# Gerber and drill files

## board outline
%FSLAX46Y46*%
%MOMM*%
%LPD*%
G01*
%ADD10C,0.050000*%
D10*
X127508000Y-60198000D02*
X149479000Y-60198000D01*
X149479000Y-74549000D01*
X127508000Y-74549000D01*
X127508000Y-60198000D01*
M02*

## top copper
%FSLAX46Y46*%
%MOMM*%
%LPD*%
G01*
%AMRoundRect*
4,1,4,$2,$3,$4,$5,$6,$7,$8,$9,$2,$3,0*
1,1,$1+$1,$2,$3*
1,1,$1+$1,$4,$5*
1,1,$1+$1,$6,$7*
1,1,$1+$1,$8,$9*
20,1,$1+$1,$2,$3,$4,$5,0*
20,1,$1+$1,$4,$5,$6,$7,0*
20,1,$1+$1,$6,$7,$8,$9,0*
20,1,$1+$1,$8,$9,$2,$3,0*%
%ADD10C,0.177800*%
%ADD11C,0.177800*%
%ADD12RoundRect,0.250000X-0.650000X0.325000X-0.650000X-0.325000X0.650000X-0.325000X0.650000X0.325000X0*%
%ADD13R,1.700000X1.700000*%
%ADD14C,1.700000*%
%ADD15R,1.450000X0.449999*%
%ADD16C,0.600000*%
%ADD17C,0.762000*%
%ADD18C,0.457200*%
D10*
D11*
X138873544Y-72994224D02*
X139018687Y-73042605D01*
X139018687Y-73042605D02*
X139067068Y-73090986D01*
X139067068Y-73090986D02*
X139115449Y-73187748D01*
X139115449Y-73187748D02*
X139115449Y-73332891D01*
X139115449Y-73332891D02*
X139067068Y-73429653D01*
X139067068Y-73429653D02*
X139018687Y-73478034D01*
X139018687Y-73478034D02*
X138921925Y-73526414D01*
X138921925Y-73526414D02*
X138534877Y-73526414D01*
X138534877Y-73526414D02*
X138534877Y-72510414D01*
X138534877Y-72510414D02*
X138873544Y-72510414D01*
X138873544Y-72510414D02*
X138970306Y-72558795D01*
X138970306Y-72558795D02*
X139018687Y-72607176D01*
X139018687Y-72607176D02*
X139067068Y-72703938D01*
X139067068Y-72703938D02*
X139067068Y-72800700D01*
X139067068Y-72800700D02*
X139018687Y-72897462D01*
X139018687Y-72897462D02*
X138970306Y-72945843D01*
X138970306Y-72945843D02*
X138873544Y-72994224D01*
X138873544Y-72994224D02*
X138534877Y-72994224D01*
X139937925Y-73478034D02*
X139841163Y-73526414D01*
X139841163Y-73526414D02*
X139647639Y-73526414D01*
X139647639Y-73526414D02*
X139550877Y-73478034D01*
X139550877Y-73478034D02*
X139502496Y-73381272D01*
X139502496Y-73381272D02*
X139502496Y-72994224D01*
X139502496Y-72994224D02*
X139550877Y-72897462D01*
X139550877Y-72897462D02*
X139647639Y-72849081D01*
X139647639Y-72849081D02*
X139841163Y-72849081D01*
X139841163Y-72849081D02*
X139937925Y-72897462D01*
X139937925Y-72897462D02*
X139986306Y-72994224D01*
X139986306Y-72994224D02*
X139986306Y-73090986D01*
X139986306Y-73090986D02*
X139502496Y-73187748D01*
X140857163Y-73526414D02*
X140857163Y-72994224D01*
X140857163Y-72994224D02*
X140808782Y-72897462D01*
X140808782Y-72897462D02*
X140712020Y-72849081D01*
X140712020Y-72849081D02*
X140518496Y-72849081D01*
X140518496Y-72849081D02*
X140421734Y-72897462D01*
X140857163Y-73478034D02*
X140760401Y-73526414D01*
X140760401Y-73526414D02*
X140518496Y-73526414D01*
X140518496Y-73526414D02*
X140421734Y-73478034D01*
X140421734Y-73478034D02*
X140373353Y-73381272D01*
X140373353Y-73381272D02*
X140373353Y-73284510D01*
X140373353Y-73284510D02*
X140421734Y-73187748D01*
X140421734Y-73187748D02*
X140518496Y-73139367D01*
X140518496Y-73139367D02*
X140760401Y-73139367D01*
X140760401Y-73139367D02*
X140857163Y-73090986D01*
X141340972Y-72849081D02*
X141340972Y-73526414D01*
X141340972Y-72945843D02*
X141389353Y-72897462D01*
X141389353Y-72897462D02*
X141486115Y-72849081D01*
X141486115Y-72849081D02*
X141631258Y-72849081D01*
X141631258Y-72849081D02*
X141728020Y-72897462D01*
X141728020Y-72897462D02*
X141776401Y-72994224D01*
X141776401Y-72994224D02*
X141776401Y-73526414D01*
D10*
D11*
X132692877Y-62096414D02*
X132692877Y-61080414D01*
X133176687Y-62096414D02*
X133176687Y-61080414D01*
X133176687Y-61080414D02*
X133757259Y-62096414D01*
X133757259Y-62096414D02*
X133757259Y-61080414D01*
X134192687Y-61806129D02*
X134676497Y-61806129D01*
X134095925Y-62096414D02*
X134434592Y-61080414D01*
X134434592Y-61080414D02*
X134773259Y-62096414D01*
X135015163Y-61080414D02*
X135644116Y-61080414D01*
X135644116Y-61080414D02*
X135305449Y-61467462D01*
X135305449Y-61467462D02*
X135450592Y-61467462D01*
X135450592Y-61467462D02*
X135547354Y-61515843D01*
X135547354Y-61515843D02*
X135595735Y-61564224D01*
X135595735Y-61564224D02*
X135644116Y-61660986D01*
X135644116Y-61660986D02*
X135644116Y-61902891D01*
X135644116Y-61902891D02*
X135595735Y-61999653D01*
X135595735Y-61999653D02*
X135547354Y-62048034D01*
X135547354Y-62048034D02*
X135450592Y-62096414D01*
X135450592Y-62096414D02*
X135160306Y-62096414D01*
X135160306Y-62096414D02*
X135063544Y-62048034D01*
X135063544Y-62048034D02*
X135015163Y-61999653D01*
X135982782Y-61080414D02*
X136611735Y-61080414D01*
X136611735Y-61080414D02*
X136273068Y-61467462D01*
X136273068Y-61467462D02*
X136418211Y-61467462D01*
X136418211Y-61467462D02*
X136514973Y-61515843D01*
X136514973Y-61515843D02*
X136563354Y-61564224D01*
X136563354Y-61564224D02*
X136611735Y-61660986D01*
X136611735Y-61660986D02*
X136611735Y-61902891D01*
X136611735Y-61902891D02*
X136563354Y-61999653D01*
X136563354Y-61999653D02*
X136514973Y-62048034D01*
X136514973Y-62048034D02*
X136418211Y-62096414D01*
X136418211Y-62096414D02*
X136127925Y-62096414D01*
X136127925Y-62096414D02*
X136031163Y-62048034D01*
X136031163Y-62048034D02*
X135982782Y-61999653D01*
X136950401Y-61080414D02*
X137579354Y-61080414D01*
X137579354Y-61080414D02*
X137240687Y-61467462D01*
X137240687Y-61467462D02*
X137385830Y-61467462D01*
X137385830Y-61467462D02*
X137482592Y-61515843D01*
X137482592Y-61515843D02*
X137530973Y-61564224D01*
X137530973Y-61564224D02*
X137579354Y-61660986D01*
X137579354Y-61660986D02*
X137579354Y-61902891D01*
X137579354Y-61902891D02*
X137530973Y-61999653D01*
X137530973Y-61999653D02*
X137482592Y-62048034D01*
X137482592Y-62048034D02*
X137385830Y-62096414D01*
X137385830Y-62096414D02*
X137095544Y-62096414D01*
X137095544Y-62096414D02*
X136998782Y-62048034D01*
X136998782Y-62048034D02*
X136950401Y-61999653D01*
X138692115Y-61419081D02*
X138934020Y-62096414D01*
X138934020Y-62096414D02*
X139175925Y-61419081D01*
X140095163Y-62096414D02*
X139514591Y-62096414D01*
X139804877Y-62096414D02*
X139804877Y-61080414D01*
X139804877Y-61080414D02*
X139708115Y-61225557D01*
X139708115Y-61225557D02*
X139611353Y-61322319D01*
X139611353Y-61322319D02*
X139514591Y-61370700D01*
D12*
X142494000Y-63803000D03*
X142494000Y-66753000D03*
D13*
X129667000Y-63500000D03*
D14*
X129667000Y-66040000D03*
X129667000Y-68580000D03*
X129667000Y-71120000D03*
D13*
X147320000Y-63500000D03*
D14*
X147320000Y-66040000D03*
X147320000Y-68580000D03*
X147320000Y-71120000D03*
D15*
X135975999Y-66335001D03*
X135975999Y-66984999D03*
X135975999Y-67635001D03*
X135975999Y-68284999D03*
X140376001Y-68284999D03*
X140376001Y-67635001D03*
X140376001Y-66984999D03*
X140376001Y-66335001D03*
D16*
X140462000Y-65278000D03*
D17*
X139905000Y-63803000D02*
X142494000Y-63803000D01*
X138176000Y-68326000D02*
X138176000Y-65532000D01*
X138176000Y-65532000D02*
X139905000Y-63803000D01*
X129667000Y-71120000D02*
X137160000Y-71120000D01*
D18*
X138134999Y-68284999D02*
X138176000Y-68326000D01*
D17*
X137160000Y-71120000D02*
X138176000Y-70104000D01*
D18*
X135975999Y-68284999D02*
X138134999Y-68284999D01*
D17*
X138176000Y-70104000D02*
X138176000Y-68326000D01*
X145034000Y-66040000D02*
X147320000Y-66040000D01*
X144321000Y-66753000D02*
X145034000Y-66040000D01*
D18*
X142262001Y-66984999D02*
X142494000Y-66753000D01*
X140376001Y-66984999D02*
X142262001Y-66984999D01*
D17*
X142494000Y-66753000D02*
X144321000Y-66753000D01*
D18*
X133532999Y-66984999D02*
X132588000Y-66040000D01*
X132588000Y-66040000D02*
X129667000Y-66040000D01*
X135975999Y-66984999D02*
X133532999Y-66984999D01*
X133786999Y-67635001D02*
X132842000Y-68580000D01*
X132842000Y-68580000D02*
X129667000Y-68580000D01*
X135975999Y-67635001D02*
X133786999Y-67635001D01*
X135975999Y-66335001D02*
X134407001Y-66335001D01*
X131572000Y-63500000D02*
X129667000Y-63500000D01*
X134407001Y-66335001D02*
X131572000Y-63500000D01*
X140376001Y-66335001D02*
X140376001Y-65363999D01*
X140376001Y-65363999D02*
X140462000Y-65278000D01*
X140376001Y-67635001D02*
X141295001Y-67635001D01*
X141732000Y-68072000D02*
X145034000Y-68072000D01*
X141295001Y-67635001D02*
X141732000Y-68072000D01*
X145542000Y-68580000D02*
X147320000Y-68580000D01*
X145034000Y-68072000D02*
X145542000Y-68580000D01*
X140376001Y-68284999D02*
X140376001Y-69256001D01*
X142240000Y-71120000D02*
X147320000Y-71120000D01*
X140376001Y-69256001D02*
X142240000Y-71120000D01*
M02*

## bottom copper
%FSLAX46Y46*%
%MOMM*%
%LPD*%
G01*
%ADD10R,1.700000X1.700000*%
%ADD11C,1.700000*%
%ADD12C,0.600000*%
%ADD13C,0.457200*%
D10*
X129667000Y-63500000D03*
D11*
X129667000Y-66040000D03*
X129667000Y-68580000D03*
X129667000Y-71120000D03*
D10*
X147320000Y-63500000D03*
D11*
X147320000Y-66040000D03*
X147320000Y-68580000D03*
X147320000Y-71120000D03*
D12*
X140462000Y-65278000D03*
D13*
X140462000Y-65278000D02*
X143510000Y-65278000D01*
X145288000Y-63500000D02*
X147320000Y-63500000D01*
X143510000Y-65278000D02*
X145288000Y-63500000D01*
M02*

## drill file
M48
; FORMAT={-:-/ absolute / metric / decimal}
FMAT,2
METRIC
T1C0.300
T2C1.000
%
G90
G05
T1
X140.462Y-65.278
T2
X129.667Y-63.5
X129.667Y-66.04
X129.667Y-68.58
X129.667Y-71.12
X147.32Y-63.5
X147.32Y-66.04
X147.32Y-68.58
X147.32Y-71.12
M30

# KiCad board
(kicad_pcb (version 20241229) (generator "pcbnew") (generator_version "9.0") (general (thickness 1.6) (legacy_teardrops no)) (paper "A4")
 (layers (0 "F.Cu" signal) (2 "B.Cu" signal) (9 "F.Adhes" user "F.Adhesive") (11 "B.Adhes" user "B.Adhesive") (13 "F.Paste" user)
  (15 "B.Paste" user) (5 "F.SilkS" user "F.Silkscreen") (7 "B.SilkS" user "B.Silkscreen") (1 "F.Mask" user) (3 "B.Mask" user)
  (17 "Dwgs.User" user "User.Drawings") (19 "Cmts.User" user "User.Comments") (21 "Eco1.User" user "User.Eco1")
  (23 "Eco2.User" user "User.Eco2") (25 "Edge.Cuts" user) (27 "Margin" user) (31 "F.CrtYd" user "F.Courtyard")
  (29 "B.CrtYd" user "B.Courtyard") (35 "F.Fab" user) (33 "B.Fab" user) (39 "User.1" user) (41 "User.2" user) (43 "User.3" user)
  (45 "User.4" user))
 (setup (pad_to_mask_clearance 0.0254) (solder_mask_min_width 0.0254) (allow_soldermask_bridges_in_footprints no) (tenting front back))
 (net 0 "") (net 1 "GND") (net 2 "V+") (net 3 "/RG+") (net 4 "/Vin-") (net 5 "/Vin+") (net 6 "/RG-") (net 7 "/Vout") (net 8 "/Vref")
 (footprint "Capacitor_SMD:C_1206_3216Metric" (layer "F.Cu") (at 142.494 65.278 -90)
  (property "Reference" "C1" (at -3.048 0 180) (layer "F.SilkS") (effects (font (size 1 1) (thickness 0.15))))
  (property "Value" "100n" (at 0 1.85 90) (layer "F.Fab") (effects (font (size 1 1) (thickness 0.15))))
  (pad "1" smd roundrect (at -1.475 0 270) (size 1.15 1.8) (layers "F.Cu" "F.Mask" "F.Paste") (roundrect_rratio 0.217391) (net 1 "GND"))
  (pad "2" smd roundrect (at 1.475 0 270) (size 1.15 1.8) (layers "F.Cu" "F.Mask" "F.Paste") (roundrect_rratio 0.217391) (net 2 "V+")))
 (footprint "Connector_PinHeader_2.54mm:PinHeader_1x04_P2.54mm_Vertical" (layer "F.Cu") (at 129.667 63.5)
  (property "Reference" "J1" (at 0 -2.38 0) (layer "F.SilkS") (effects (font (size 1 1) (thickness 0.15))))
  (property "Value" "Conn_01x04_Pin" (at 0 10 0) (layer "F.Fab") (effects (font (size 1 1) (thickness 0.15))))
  (pad "1" thru_hole rect (at 0 0) (size 1.7 1.7) (drill 1) (layers "*.Cu" "*.Mask") (remove_unused_layers no) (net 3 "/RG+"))
  (pad "2" thru_hole circle (at 0 2.54) (size 1.7 1.7) (drill 1) (layers "*.Cu" "*.Mask") (remove_unused_layers no) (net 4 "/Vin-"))
  (pad "3" thru_hole circle (at 0 5.08) (size 1.7 1.7) (drill 1) (layers "*.Cu" "*.Mask") (remove_unused_layers no) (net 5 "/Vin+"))
  (pad "4" thru_hole circle (at 0 7.62) (size 1.7 1.7) (drill 1) (layers "*.Cu" "*.Mask") (remove_unused_layers no) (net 1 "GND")))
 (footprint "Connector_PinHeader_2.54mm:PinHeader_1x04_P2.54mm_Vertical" (layer "F.Cu") (at 147.32 63.5)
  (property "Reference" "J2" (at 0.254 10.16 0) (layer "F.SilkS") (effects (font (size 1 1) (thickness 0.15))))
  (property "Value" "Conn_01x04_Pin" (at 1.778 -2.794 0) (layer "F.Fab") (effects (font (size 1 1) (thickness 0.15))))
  (pad "1" thru_hole rect (at 0 0) (size 1.7 1.7) (drill 1) (layers "*.Cu" "*.Mask") (remove_unused_layers no) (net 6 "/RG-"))
  (pad "2" thru_hole circle (at 0 2.54) (size 1.7 1.7) (drill 1) (layers "*.Cu" "*.Mask") (remove_unused_layers no) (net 2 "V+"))
  (pad "3" thru_hole circle (at 0 5.08) (size 1.7 1.7) (drill 1) (layers "*.Cu" "*.Mask") (remove_unused_layers no) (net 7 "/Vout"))
  (pad "4" thru_hole circle (at 0 7.62) (size 1.7 1.7) (drill 1) (layers "*.Cu" "*.Mask") (remove_unused_layers no) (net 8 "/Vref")))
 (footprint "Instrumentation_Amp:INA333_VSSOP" (layer "F.Cu") (at 138.176 67.31)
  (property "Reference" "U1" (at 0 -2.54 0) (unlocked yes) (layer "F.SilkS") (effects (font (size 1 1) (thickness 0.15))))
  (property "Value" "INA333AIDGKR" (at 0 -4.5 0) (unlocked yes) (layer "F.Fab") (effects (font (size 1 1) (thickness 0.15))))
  (pad "1" smd rect (at -2.200001 -0.974999) (size 1.45 0.449999) (layers "F.Cu" "F.Mask" "F.Paste") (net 3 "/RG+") (solder_mask_margin 0)
   (solder_paste_margin 0) (clearance 0))
  (pad "2" smd rect (at -2.200001 -0.325001) (size 1.45 0.449999) (layers "F.Cu" "F.Mask" "F.Paste") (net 4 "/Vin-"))
  (pad "3" smd rect (at -2.200001 0.325001) (size 1.45 0.449999) (layers "F.Cu" "F.Mask" "F.Paste") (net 5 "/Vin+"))
  (pad "4" smd rect (at -2.200001 0.974999) (size 1.45 0.449999) (layers "F.Cu" "F.Mask" "F.Paste") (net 1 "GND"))
  (pad "5" smd rect (at 2.200001 0.974999) (size 1.45 0.449999) (layers "F.Cu" "F.Mask" "F.Paste") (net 8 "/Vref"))
  (pad "6" smd rect (at 2.200001 0.325001) (size 1.45 0.449999) (layers "F.Cu" "F.Mask" "F.Paste") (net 7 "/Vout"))
  (pad "7" smd rect (at 2.200001 -0.325001) (size 1.45 0.449999) (layers "F.Cu" "F.Mask" "F.Paste") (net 2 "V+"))
  (pad "8" smd rect (at 2.200001 -0.974999) (size 1.45 0.449999) (layers "F.Cu" "F.Mask" "F.Paste") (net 6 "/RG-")))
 (gr_rect (start 127.508 60.198) (end 149.479 74.549) (stroke (width 0.05) (type solid)) (fill no) (layer "Edge.Cuts"))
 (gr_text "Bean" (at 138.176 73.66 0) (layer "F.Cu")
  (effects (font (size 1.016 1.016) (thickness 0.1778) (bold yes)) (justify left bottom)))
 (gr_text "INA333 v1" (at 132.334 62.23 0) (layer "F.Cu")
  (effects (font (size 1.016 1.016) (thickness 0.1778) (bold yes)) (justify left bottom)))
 (segment (start 139.905 63.803) (end 142.494 63.803) (width 0.762) (layer "F.Cu") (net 1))
 (segment (start 138.176 68.326) (end 138.176 65.532) (width 0.762) (layer "F.Cu") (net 1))
 (segment (start 138.176 65.532) (end 139.905 63.803) (width 0.762) (layer "F.Cu") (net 1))
 (segment (start 129.667 71.12) (end 137.16 71.12) (width 0.762) (layer "F.Cu") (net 1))
 (segment (start 138.134999 68.284999) (end 138.176 68.326) (width 0.4572) (layer "F.Cu") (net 1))
 (segment (start 137.16 71.12) (end 138.176 70.104) (width 0.762) (layer "F.Cu") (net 1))
 (segment (start 135.975999 68.284999) (end 138.134999 68.284999) (width 0.4572) (layer "F.Cu") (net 1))
 (segment (start 138.176 70.104) (end 138.176 68.326) (width 0.762) (layer "F.Cu") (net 1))
 (segment (start 145.034 66.04) (end 147.32 66.04) (width 0.762) (layer "F.Cu") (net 2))
 (segment (start 144.321 66.753) (end 145.034 66.04) (width 0.762) (layer "F.Cu") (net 2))
 (segment (start 142.262001 66.984999) (end 142.494 66.753) (width 0.4572) (layer "F.Cu") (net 2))
 (segment (start 140.376001 66.984999) (end 142.262001 66.984999) (width 0.4572) (layer "F.Cu") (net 2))
 (segment (start 142.494 66.753) (end 144.321 66.753) (width 0.762) (layer "F.Cu") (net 2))
 (segment (start 133.532999 66.984999) (end 132.588 66.04) (width 0.4572) (layer "F.Cu") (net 4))
 (segment (start 132.588 66.04) (end 129.667 66.04) (width 0.4572) (layer "F.Cu") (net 4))
 (segment (start 135.975999 66.984999) (end 133.532999 66.984999) (width 0.4572) (layer "F.Cu") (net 4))
 (segment (start 133.786999 67.635001) (end 132.842 68.58) (width 0.4572) (layer "F.Cu") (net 5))
 (segment (start 132.842 68.58) (end 129.667 68.58) (width 0.4572) (layer "F.Cu") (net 5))
 (segment (start 135.975999 67.635001) (end 133.786999 67.635001) (width 0.4572) (layer "F.Cu") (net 5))
 (segment (start 135.975999 66.335001) (end 134.407001 66.335001) (width 0.4572) (layer "F.Cu") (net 3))
 (segment (start 131.572 63.5) (end 129.667 63.5) (width 0.4572) (layer "F.Cu") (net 3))
 (segment (start 134.407001 66.335001) (end 131.572 63.5) (width 0.4572) (layer "F.Cu") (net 3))
 (segment (start 140.376001 66.335001) (end 140.376001 65.363999) (width 0.4572) (layer "F.Cu") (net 6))
 (segment (start 140.376001 65.363999) (end 140.462 65.278) (width 0.4572) (layer "F.Cu") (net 6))
 (via (at 140.462 65.278) (size 0.6) (drill 0.3) (layers "F.Cu" "B.Cu") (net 6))
 (segment (start 140.462 65.278) (end 143.51 65.278) (width 0.4572) (layer "B.Cu") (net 6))
 (segment (start 145.288 63.5) (end 147.32 63.5) (width 0.4572) (layer "B.Cu") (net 6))
 (segment (start 143.51 65.278) (end 145.288 63.5) (width 0.4572) (layer "B.Cu") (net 6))
 (segment (start 140.376001 67.635001) (end 141.295001 67.635001) (width 0.4572) (layer "F.Cu") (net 7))
 (segment (start 141.732 68.072) (end 145.034 68.072) (width 0.4572) (layer "F.Cu") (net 7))
 (segment (start 141.295001 67.635001) (end 141.732 68.072) (width 0.4572) (layer "F.Cu") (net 7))
 (segment (start 145.542 68.58) (end 147.32 68.58) (width 0.4572) (layer "F.Cu") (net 7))
 (segment (start 145.034 68.072) (end 145.542 68.58) (width 0.4572) (layer "F.Cu") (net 7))
 (segment (start 140.376001 68.284999) (end 140.376001 69.256001) (width 0.4572) (layer "F.Cu") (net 8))
 (segment (start 142.24 71.12) (end 147.32 71.12) (width 0.4572) (layer "F.Cu") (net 8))
 (segment (start 140.376001 69.256001) (end 142.24 71.12) (width 0.4572) (layer "F.Cu") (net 8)))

